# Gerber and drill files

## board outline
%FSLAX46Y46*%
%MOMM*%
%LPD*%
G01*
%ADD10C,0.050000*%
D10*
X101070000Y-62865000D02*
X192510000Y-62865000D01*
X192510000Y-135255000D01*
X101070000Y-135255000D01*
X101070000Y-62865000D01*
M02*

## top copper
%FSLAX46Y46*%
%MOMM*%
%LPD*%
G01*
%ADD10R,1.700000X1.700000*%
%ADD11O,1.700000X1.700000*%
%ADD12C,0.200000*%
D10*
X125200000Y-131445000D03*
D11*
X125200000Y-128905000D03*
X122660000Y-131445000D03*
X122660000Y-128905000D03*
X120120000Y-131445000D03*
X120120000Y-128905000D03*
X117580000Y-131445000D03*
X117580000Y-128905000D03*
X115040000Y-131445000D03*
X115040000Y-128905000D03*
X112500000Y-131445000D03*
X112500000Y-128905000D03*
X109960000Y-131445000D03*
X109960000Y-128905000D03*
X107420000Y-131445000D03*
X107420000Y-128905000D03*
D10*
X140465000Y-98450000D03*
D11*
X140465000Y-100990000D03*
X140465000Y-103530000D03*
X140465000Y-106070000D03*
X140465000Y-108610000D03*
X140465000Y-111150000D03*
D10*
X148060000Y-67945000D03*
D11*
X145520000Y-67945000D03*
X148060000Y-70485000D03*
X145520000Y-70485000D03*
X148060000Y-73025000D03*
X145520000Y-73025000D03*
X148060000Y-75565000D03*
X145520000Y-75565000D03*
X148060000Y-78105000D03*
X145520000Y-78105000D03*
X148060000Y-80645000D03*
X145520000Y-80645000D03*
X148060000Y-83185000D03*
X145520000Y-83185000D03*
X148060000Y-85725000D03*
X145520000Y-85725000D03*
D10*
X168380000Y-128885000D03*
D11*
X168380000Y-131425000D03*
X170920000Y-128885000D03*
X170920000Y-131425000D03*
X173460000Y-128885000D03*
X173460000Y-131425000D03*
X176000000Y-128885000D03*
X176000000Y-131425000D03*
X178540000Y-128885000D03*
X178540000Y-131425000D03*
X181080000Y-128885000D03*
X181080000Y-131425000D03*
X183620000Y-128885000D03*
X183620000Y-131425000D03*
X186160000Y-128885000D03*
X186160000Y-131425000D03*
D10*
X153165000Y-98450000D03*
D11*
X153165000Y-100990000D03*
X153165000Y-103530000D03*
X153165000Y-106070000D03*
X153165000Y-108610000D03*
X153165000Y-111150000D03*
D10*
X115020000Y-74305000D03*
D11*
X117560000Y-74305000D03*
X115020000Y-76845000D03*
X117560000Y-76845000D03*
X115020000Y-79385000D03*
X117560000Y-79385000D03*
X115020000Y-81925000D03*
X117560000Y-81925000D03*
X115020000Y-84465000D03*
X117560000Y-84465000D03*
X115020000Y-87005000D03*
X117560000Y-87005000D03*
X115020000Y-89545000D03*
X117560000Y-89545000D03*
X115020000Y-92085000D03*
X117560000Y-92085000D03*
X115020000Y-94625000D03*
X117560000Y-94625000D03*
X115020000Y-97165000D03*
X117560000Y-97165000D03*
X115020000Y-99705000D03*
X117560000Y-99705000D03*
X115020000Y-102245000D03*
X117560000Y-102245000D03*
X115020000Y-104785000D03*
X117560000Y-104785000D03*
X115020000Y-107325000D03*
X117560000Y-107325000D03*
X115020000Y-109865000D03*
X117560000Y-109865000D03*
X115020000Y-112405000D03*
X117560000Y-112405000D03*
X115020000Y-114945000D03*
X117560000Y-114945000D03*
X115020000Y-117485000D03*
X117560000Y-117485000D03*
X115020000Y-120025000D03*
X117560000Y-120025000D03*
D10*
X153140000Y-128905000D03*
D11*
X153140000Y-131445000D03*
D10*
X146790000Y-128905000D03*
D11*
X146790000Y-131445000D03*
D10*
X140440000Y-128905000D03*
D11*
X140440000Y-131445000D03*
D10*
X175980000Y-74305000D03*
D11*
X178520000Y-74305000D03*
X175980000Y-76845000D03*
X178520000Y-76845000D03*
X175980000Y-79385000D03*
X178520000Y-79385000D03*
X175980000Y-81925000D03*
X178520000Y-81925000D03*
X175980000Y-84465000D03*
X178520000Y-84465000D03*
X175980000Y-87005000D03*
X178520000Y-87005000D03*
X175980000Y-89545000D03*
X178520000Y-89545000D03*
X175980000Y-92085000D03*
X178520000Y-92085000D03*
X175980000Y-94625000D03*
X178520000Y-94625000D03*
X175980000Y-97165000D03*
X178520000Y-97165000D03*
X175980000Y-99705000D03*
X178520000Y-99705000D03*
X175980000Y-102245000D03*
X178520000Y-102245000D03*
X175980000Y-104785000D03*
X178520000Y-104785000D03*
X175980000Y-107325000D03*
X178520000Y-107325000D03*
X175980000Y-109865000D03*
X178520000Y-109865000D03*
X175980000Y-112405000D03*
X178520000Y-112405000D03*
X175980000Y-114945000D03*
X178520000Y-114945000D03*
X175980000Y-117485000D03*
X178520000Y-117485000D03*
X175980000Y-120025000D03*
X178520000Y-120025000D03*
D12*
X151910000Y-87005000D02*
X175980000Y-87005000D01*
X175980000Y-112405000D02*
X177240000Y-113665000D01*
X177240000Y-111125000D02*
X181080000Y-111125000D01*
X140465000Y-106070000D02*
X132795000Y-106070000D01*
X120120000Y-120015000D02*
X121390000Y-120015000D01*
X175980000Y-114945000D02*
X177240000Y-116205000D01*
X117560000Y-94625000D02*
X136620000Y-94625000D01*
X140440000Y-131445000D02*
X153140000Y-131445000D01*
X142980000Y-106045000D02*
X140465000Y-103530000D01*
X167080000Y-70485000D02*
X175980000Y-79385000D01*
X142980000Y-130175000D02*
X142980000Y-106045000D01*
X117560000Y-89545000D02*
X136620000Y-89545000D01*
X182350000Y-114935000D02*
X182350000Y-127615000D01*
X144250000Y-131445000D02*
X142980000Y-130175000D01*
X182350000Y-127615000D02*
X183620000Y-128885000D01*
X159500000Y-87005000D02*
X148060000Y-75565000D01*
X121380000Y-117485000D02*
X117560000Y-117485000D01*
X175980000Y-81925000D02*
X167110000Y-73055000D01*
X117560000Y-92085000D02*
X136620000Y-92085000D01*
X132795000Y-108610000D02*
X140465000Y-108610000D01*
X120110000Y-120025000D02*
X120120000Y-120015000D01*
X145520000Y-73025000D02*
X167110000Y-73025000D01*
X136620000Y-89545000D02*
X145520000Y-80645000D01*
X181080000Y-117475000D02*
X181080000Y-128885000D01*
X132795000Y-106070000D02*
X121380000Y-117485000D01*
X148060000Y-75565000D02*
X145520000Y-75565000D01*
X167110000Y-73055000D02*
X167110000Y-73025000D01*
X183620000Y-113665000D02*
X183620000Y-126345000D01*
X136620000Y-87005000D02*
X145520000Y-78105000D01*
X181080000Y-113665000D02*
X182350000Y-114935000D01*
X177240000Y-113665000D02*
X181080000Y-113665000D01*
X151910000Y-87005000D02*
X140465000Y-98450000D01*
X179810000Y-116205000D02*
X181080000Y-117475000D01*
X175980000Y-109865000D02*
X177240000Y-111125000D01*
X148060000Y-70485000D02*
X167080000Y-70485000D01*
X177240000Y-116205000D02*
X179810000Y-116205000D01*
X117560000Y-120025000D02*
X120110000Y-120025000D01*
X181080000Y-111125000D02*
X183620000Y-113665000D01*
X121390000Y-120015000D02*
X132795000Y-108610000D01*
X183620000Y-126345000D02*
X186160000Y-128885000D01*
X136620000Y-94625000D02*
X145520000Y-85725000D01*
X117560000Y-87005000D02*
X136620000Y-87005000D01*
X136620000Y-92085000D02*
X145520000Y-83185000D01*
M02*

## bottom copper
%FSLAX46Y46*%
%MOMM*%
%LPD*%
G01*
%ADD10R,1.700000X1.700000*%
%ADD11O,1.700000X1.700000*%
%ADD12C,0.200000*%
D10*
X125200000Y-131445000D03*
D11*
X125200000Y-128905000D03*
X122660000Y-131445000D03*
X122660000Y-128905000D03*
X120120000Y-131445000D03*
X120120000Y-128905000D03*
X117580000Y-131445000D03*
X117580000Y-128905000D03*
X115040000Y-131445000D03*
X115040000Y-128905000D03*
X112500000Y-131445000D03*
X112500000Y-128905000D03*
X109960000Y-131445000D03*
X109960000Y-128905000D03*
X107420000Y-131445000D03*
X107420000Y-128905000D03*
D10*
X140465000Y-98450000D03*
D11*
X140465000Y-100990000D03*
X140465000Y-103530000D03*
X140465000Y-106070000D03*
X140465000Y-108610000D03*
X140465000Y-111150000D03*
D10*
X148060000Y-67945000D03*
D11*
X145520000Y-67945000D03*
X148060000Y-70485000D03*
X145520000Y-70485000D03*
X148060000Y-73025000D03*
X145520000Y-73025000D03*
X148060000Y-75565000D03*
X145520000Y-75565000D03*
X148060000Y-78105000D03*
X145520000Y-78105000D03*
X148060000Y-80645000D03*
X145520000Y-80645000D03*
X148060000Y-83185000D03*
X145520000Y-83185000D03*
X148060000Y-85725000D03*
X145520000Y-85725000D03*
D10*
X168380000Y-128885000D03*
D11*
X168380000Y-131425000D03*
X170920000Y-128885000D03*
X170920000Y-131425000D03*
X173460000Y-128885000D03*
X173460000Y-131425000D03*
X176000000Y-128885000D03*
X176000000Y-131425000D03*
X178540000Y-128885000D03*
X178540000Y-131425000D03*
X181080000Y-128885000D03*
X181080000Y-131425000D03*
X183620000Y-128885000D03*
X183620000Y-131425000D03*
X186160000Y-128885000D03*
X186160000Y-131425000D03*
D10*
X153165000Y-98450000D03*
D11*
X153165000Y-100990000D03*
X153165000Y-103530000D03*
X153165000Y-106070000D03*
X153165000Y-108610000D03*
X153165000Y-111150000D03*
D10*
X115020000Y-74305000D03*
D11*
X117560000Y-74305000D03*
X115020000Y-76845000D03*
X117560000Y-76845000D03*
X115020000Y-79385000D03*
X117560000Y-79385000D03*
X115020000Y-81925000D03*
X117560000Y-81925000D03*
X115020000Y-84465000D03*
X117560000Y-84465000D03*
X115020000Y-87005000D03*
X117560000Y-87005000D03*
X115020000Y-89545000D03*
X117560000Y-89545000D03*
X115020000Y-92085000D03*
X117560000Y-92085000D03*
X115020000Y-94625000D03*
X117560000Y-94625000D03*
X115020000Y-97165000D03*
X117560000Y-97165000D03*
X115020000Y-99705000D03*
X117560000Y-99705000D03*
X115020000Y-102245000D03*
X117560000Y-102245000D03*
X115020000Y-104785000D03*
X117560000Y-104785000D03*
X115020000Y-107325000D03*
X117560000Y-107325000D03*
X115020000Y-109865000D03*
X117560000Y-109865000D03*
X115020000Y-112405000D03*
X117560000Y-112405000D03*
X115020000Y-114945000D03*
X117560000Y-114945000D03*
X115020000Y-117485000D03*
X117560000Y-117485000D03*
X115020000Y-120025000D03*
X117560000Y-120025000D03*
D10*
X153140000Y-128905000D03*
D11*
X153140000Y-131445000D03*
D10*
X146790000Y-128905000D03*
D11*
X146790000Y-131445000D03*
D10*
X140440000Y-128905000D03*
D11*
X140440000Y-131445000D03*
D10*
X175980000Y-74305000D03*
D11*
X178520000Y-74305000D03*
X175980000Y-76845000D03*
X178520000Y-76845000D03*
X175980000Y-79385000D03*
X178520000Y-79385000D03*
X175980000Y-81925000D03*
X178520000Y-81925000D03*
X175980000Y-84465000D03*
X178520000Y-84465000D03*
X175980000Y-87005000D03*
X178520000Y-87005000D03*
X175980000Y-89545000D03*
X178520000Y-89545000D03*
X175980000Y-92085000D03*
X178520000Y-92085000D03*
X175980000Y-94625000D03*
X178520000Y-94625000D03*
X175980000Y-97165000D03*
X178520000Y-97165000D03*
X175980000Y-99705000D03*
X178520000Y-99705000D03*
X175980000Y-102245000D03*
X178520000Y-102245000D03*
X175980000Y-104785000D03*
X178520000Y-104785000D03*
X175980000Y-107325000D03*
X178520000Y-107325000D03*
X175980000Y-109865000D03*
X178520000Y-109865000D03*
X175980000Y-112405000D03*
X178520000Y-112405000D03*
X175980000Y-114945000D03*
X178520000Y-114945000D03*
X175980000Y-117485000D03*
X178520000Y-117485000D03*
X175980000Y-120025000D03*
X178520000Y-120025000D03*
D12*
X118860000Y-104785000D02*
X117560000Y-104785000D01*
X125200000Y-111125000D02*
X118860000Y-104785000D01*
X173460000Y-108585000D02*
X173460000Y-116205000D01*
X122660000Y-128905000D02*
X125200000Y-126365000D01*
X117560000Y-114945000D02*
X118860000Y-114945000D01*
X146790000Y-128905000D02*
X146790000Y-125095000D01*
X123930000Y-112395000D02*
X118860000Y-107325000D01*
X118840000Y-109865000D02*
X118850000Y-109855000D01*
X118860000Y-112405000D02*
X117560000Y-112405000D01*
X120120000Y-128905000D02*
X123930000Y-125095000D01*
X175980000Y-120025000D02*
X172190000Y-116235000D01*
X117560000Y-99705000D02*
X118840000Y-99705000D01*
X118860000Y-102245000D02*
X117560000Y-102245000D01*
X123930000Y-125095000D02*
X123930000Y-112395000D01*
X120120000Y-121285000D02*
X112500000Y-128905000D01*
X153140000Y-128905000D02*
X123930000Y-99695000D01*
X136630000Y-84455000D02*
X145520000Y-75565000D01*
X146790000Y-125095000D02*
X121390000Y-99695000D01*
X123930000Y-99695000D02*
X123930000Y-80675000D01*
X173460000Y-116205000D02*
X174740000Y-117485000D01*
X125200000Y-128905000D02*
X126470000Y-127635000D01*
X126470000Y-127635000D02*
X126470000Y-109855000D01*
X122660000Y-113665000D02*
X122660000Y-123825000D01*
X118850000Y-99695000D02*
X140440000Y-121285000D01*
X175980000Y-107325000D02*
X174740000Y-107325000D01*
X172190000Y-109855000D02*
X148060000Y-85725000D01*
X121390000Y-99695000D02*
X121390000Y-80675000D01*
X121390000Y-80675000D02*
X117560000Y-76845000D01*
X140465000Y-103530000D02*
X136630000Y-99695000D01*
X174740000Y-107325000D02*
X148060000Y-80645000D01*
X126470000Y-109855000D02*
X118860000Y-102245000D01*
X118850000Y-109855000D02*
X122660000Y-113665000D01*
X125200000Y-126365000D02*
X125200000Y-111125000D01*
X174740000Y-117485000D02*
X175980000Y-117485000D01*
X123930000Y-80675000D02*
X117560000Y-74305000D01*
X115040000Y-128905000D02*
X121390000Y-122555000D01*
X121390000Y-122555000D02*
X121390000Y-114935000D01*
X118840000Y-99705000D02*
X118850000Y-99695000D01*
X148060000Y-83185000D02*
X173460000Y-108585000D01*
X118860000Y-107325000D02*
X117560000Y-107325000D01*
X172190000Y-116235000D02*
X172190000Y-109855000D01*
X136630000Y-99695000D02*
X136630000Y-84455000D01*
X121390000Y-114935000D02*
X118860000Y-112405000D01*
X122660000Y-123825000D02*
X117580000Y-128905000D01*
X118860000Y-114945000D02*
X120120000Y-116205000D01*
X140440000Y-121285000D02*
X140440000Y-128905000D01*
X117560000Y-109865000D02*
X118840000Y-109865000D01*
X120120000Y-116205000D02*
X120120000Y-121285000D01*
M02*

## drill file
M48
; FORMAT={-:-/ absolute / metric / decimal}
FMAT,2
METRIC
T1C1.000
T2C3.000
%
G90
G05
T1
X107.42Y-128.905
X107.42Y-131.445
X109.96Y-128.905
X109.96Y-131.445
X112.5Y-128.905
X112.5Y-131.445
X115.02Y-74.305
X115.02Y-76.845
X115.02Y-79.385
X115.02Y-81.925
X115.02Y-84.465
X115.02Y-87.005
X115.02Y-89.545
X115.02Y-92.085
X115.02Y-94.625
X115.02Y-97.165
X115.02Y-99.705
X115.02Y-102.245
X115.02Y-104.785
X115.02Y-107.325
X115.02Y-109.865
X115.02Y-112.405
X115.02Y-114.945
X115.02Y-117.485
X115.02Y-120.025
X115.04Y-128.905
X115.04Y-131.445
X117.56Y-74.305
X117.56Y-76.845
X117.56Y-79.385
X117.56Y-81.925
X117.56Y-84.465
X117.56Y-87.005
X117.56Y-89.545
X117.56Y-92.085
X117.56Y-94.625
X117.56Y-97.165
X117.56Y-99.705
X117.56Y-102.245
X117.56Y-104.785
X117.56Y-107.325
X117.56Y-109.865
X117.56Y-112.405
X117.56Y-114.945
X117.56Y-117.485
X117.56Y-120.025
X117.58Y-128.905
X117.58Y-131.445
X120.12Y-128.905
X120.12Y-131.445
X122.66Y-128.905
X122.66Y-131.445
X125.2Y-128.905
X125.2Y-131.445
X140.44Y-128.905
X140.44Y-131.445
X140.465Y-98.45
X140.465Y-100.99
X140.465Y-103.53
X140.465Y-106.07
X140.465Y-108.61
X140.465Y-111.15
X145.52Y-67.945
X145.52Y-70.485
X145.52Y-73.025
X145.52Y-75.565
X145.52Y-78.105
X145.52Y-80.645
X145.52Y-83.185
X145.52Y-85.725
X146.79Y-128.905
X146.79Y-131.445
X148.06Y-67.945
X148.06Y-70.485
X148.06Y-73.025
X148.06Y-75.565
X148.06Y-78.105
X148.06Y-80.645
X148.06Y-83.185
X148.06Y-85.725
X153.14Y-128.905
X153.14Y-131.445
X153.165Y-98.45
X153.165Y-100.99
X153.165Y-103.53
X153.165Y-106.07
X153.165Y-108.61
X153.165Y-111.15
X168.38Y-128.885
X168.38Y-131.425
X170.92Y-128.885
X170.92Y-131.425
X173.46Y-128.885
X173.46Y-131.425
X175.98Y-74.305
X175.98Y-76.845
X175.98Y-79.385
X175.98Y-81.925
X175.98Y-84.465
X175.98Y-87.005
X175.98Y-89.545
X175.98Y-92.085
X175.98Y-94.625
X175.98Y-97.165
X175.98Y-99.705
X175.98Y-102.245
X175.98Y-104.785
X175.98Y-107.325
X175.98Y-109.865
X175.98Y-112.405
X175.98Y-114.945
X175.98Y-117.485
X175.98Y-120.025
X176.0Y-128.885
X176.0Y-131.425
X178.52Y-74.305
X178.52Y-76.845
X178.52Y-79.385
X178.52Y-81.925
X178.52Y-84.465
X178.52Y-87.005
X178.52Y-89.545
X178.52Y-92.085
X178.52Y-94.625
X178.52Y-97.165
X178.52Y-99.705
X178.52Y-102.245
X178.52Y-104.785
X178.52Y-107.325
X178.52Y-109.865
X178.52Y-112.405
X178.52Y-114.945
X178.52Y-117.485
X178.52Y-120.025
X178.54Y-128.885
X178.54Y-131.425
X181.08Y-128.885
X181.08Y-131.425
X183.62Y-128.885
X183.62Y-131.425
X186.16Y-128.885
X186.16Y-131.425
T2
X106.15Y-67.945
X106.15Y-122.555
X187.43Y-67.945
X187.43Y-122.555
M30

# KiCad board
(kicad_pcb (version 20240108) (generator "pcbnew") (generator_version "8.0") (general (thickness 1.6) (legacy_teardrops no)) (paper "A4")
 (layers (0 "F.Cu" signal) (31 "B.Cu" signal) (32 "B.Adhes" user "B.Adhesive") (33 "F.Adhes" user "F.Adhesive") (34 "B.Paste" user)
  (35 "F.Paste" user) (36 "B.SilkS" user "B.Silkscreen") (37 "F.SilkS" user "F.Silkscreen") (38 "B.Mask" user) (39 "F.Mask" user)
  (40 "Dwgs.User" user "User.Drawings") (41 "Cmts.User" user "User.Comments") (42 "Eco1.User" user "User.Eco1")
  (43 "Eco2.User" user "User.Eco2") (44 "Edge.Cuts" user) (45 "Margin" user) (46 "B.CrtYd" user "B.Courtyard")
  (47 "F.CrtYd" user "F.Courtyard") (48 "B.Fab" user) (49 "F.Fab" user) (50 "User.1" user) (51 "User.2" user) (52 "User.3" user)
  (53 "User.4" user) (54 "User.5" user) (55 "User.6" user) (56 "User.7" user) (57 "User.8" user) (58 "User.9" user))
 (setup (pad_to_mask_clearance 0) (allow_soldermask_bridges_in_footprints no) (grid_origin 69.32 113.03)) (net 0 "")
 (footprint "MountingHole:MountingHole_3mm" (layer "F.Cu") (at 106.15 67.945)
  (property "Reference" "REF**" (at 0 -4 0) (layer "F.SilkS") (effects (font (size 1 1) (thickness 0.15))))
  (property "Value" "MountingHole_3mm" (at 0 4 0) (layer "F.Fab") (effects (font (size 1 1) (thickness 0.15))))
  (pad "" np_thru_hole circle (at 0 0) (size 3 3) (drill 3) (layers "*.Cu" "*.Mask")))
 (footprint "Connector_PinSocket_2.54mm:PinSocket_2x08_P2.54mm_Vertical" (layer "F.Cu") (at 125.2 131.445 -90)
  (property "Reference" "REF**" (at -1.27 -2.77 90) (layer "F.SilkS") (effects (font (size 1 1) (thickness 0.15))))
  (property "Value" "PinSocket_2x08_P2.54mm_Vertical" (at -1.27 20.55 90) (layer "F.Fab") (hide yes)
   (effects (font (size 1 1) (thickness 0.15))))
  (pad "1" thru_hole rect (at 0 0 270) (size 1.7 1.7) (drill 1) (layers "*.Cu" "*.Mask") (remove_unused_layers no))
  (pad "2" thru_hole oval (at -2.54 0 270) (size 1.7 1.7) (drill 1) (layers "*.Cu" "*.Mask") (remove_unused_layers no))
  (pad "3" thru_hole oval (at 0 2.54 270) (size 1.7 1.7) (drill 1) (layers "*.Cu" "*.Mask") (remove_unused_layers no))
  (pad "4" thru_hole oval (at -2.54 2.54 270) (size 1.7 1.7) (drill 1) (layers "*.Cu" "*.Mask") (remove_unused_layers no))
  (pad "5" thru_hole oval (at 0 5.08 270) (size 1.7 1.7) (drill 1) (layers "*.Cu" "*.Mask") (remove_unused_layers no))
  (pad "6" thru_hole oval (at -2.54 5.08 270) (size 1.7 1.7) (drill 1) (layers "*.Cu" "*.Mask") (remove_unused_layers no))
  (pad "7" thru_hole oval (at 0 7.62 270) (size 1.7 1.7) (drill 1) (layers "*.Cu" "*.Mask") (remove_unused_layers no))
  (pad "8" thru_hole oval (at -2.54 7.62 270) (size 1.7 1.7) (drill 1) (layers "*.Cu" "*.Mask") (remove_unused_layers no))
  (pad "9" thru_hole oval (at 0 10.16 270) (size 1.7 1.7) (drill 1) (layers "*.Cu" "*.Mask") (remove_unused_layers no))
  (pad "10" thru_hole oval (at -2.54 10.16 270) (size 1.7 1.7) (drill 1) (layers "*.Cu" "*.Mask") (remove_unused_layers no))
  (pad "11" thru_hole oval (at 0 12.7 270) (size 1.7 1.7) (drill 1) (layers "*.Cu" "*.Mask") (remove_unused_layers no))
  (pad "12" thru_hole oval (at -2.54 12.7 270) (size 1.7 1.7) (drill 1) (layers "*.Cu" "*.Mask") (remove_unused_layers no))
  (pad "13" thru_hole oval (at 0 15.24 270) (size 1.7 1.7) (drill 1) (layers "*.Cu" "*.Mask") (remove_unused_layers no))
  (pad "14" thru_hole oval (at -2.54 15.24 270) (size 1.7 1.7) (drill 1) (layers "*.Cu" "*.Mask") (remove_unused_layers no))
  (pad "15" thru_hole oval (at 0 17.78 270) (size 1.7 1.7) (drill 1) (layers "*.Cu" "*.Mask") (remove_unused_layers no))
  (pad "16" thru_hole oval (at -2.54 17.78 270) (size 1.7 1.7) (drill 1) (layers "*.Cu" "*.Mask") (remove_unused_layers no)))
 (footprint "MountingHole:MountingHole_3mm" (layer "F.Cu") (at 187.43 122.555)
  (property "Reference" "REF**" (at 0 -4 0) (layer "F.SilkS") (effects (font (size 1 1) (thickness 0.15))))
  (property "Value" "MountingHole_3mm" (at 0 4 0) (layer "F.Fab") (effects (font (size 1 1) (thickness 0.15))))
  (pad "" np_thru_hole circle (at 0 0) (size 3 3) (drill 3) (layers "*.Cu" "*.Mask")))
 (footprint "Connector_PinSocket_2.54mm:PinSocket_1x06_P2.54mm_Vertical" (layer "F.Cu") (at 140.465 98.45)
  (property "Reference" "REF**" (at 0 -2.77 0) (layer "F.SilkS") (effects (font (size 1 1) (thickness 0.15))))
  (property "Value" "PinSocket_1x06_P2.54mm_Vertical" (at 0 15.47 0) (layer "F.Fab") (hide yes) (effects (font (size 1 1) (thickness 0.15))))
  (pad "1" thru_hole rect (at 0 0) (size 1.7 1.7) (drill 1) (layers "*.Cu" "*.Mask") (remove_unused_layers no))
  (pad "2" thru_hole oval (at 0 2.54) (size 1.7 1.7) (drill 1) (layers "*.Cu" "*.Mask") (remove_unused_layers no))
  (pad "3" thru_hole oval (at 0 5.08) (size 1.7 1.7) (drill 1) (layers "*.Cu" "*.Mask") (remove_unused_layers no))
  (pad "4" thru_hole oval (at 0 7.62) (size 1.7 1.7) (drill 1) (layers "*.Cu" "*.Mask") (remove_unused_layers no))
  (pad "5" thru_hole oval (at 0 10.16) (size 1.7 1.7) (drill 1) (layers "*.Cu" "*.Mask") (remove_unused_layers no))
  (pad "6" thru_hole oval (at 0 12.7) (size 1.7 1.7) (drill 1) (layers "*.Cu" "*.Mask") (remove_unused_layers no)))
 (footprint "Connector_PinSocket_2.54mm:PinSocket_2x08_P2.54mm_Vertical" (layer "F.Cu") (at 148.06 67.945)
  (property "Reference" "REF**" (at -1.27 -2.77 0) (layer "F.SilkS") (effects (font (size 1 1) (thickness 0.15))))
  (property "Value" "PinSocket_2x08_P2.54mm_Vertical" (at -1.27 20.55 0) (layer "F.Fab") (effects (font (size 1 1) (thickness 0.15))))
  (pad "1" thru_hole rect (at 0 0) (size 1.7 1.7) (drill 1) (layers "*.Cu" "*.Mask") (remove_unused_layers no))
  (pad "2" thru_hole oval (at -2.54 0) (size 1.7 1.7) (drill 1) (layers "*.Cu" "*.Mask") (remove_unused_layers no))
  (pad "3" thru_hole oval (at 0 2.54) (size 1.7 1.7) (drill 1) (layers "*.Cu" "*.Mask") (remove_unused_layers no))
  (pad "4" thru_hole oval (at -2.54 2.54) (size 1.7 1.7) (drill 1) (layers "*.Cu" "*.Mask") (remove_unused_layers no))
  (pad "5" thru_hole oval (at 0 5.08) (size 1.7 1.7) (drill 1) (layers "*.Cu" "*.Mask") (remove_unused_layers no))
  (pad "6" thru_hole oval (at -2.54 5.08) (size 1.7 1.7) (drill 1) (layers "*.Cu" "*.Mask") (remove_unused_layers no))
  (pad "7" thru_hole oval (at 0 7.62) (size 1.7 1.7) (drill 1) (layers "*.Cu" "*.Mask") (remove_unused_layers no))
  (pad "8" thru_hole oval (at -2.54 7.62) (size 1.7 1.7) (drill 1) (layers "*.Cu" "*.Mask") (remove_unused_layers no))
  (pad "9" thru_hole oval (at 0 10.16) (size 1.7 1.7) (drill 1) (layers "*.Cu" "*.Mask") (remove_unused_layers no))
  (pad "10" thru_hole oval (at -2.54 10.16) (size 1.7 1.7) (drill 1) (layers "*.Cu" "*.Mask") (remove_unused_layers no))
  (pad "11" thru_hole oval (at 0 12.7) (size 1.7 1.7) (drill 1) (layers "*.Cu" "*.Mask") (remove_unused_layers no))
  (pad "12" thru_hole oval (at -2.54 12.7) (size 1.7 1.7) (drill 1) (layers "*.Cu" "*.Mask") (remove_unused_layers no))
  (pad "13" thru_hole oval (at 0 15.24) (size 1.7 1.7) (drill 1) (layers "*.Cu" "*.Mask") (remove_unused_layers no))
  (pad "14" thru_hole oval (at -2.54 15.24) (size 1.7 1.7) (drill 1) (layers "*.Cu" "*.Mask") (remove_unused_layers no))
  (pad "15" thru_hole oval (at 0 17.78) (size 1.7 1.7) (drill 1) (layers "*.Cu" "*.Mask") (remove_unused_layers no))
  (pad "16" thru_hole oval (at -2.54 17.78) (size 1.7 1.7) (drill 1) (layers "*.Cu" "*.Mask") (remove_unused_layers no)))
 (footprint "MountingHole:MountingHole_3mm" (layer "F.Cu") (at 106.15 122.555)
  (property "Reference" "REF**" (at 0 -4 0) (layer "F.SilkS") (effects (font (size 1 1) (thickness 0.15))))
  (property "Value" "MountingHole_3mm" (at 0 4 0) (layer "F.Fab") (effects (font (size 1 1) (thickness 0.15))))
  (pad "" np_thru_hole circle (at 0 0) (size 3 3) (drill 3) (layers "*.Cu" "*.Mask")))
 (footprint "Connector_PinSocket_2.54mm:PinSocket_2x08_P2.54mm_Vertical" (layer "F.Cu") (at 168.38 128.885 90)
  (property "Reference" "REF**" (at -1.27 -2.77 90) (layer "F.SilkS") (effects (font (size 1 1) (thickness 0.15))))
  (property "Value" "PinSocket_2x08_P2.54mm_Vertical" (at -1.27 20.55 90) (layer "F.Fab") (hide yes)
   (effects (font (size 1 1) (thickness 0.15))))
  (pad "1" thru_hole rect (at 0 0 90) (size 1.7 1.7) (drill 1) (layers "*.Cu" "*.Mask") (remove_unused_layers no))
  (pad "2" thru_hole oval (at -2.54 0 90) (size 1.7 1.7) (drill 1) (layers "*.Cu" "*.Mask") (remove_unused_layers no))
  (pad "3" thru_hole oval (at 0 2.54 90) (size 1.7 1.7) (drill 1) (layers "*.Cu" "*.Mask") (remove_unused_layers no))
  (pad "4" thru_hole oval (at -2.54 2.54 90) (size 1.7 1.7) (drill 1) (layers "*.Cu" "*.Mask") (remove_unused_layers no))
  (pad "5" thru_hole oval (at 0 5.08 90) (size 1.7 1.7) (drill 1) (layers "*.Cu" "*.Mask") (remove_unused_layers no))
  (pad "6" thru_hole oval (at -2.54 5.08 90) (size 1.7 1.7) (drill 1) (layers "*.Cu" "*.Mask") (remove_unused_layers no))
  (pad "7" thru_hole oval (at 0 7.62 90) (size 1.7 1.7) (drill 1) (layers "*.Cu" "*.Mask") (remove_unused_layers no))
  (pad "8" thru_hole oval (at -2.54 7.62 90) (size 1.7 1.7) (drill 1) (layers "*.Cu" "*.Mask") (remove_unused_layers no))
  (pad "9" thru_hole oval (at 0 10.16 90) (size 1.7 1.7) (drill 1) (layers "*.Cu" "*.Mask") (remove_unused_layers no))
  (pad "10" thru_hole oval (at -2.54 10.16 90) (size 1.7 1.7) (drill 1) (layers "*.Cu" "*.Mask") (remove_unused_layers no))
  (pad "11" thru_hole oval (at 0 12.7 90) (size 1.7 1.7) (drill 1) (layers "*.Cu" "*.Mask") (remove_unused_layers no))
  (pad "12" thru_hole oval (at -2.54 12.7 90) (size 1.7 1.7) (drill 1) (layers "*.Cu" "*.Mask") (remove_unused_layers no))
  (pad "13" thru_hole oval (at 0 15.24 90) (size 1.7 1.7) (drill 1) (layers "*.Cu" "*.Mask") (remove_unused_layers no))
  (pad "14" thru_hole oval (at -2.54 15.24 90) (size 1.7 1.7) (drill 1) (layers "*.Cu" "*.Mask") (remove_unused_layers no))
  (pad "15" thru_hole oval (at 0 17.78 90) (size 1.7 1.7) (drill 1) (layers "*.Cu" "*.Mask") (remove_unused_layers no))
  (pad "16" thru_hole oval (at -2.54 17.78 90) (size 1.7 1.7) (drill 1) (layers "*.Cu" "*.Mask") (remove_unused_layers no)))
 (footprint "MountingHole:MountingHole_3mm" (layer "F.Cu") (at 187.43 67.945)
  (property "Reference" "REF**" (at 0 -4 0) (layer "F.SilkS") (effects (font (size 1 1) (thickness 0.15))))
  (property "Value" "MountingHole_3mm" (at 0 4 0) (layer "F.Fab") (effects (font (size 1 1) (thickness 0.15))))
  (pad "" np_thru_hole circle (at 0 0) (size 3 3) (drill 3) (layers "*.Cu" "*.Mask")))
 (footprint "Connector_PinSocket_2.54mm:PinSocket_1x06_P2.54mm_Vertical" (layer "F.Cu") (at 153.165 98.45)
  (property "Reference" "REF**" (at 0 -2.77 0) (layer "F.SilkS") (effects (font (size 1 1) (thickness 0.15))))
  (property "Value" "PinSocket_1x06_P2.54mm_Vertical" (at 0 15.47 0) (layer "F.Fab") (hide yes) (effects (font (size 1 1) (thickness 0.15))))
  (pad "1" thru_hole rect (at 0 0) (size 1.7 1.7) (drill 1) (layers "*.Cu" "*.Mask") (remove_unused_layers no))
  (pad "2" thru_hole oval (at 0 2.54) (size 1.7 1.7) (drill 1) (layers "*.Cu" "*.Mask") (remove_unused_layers no))
  (pad "3" thru_hole oval (at 0 5.08) (size 1.7 1.7) (drill 1) (layers "*.Cu" "*.Mask") (remove_unused_layers no))
  (pad "4" thru_hole oval (at 0 7.62) (size 1.7 1.7) (drill 1) (layers "*.Cu" "*.Mask") (remove_unused_layers no))
  (pad "5" thru_hole oval (at 0 10.16) (size 1.7 1.7) (drill 1) (layers "*.Cu" "*.Mask") (remove_unused_layers no))
  (pad "6" thru_hole oval (at 0 12.7) (size 1.7 1.7) (drill 1) (layers "*.Cu" "*.Mask") (remove_unused_layers no)))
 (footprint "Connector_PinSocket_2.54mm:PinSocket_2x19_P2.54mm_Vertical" (layer "B.Cu") (at 115.02 74.305 180)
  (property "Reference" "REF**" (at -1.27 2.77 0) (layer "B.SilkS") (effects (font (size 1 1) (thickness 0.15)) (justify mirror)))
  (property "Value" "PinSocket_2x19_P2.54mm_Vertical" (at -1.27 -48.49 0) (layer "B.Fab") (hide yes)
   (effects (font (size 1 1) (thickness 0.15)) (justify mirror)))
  (pad "1" thru_hole rect (at 0 0 180) (size 1.7 1.7) (drill 1) (layers "*.Cu" "*.Mask") (remove_unused_layers no))
  (pad "2" thru_hole oval (at -2.54 0 180) (size 1.7 1.7) (drill 1) (layers "*.Cu" "*.Mask") (remove_unused_layers no))
  (pad "3" thru_hole oval (at 0 -2.54 180) (size 1.7 1.7) (drill 1) (layers "*.Cu" "*.Mask") (remove_unused_layers no))
  (pad "4" thru_hole oval (at -2.54 -2.54 180) (size 1.7 1.7) (drill 1) (layers "*.Cu" "*.Mask") (remove_unused_layers no))
  (pad "5" thru_hole oval (at 0 -5.08 180) (size 1.7 1.7) (drill 1) (layers "*.Cu" "*.Mask") (remove_unused_layers no))
  (pad "6" thru_hole oval (at -2.54 -5.08 180) (size 1.7 1.7) (drill 1) (layers "*.Cu" "*.Mask") (remove_unused_layers no))
  (pad "7" thru_hole oval (at 0 -7.62 180) (size 1.7 1.7) (drill 1) (layers "*.Cu" "*.Mask") (remove_unused_layers no))
  (pad "8" thru_hole oval (at -2.54 -7.62 180) (size 1.7 1.7) (drill 1) (layers "*.Cu" "*.Mask") (remove_unused_layers no))
  (pad "9" thru_hole oval (at 0 -10.16 180) (size 1.7 1.7) (drill 1) (layers "*.Cu" "*.Mask") (remove_unused_layers no))
  (pad "10" thru_hole oval (at -2.54 -10.16 180) (size 1.7 1.7) (drill 1) (layers "*.Cu" "*.Mask") (remove_unused_layers no))
  (pad "11" thru_hole oval (at 0 -12.7 180) (size 1.7 1.7) (drill 1) (layers "*.Cu" "*.Mask") (remove_unused_layers no))
  (pad "12" thru_hole oval (at -2.54 -12.7 180) (size 1.7 1.7) (drill 1) (layers "*.Cu" "*.Mask") (remove_unused_layers no))
  (pad "13" thru_hole oval (at 0 -15.24 180) (size 1.7 1.7) (drill 1) (layers "*.Cu" "*.Mask") (remove_unused_layers no))
  (pad "14" thru_hole oval (at -2.54 -15.24 180) (size 1.7 1.7) (drill 1) (layers "*.Cu" "*.Mask") (remove_unused_layers no))
  (pad "15" thru_hole oval (at 0 -17.78 180) (size 1.7 1.7) (drill 1) (layers "*.Cu" "*.Mask") (remove_unused_layers no))
  (pad "16" thru_hole oval (at -2.54 -17.78 180) (size 1.7 1.7) (drill 1) (layers "*.Cu" "*.Mask") (remove_unused_layers no))
  (pad "17" thru_hole oval (at 0 -20.32 180) (size 1.7 1.7) (drill 1) (layers "*.Cu" "*.Mask") (remove_unused_layers no))
  (pad "18" thru_hole oval (at -2.54 -20.32 180) (size 1.7 1.7) (drill 1) (layers "*.Cu" "*.Mask") (remove_unused_layers no))
  (pad "19" thru_hole oval (at 0 -22.86 180) (size 1.7 1.7) (drill 1) (layers "*.Cu" "*.Mask") (remove_unused_layers no))
  (pad "20" thru_hole oval (at -2.54 -22.86 180) (size 1.7 1.7) (drill 1) (layers "*.Cu" "*.Mask") (remove_unused_layers no))
  (pad "21" thru_hole oval (at 0 -25.4 180) (size 1.7 1.7) (drill 1) (layers "*.Cu" "*.Mask") (remove_unused_layers no))
  (pad "22" thru_hole oval (at -2.54 -25.4 180) (size 1.7 1.7) (drill 1) (layers "*.Cu" "*.Mask") (remove_unused_layers no))
  (pad "23" thru_hole oval (at 0 -27.94 180) (size 1.7 1.7) (drill 1) (layers "*.Cu" "*.Mask") (remove_unused_layers no))
  (pad "24" thru_hole oval (at -2.54 -27.94 180) (size 1.7 1.7) (drill 1) (layers "*.Cu" "*.Mask") (remove_unused_layers no))
  (pad "25" thru_hole oval (at 0 -30.48 180) (size 1.7 1.7) (drill 1) (layers "*.Cu" "*.Mask") (remove_unused_layers no))
  (pad "26" thru_hole oval (at -2.54 -30.48 180) (size 1.7 1.7) (drill 1) (layers "*.Cu" "*.Mask") (remove_unused_layers no))
  (pad "27" thru_hole oval (at 0 -33.02 180) (size 1.7 1.7) (drill 1) (layers "*.Cu" "*.Mask") (remove_unused_layers no))
  (pad "28" thru_hole oval (at -2.54 -33.02 180) (size 1.7 1.7) (drill 1) (layers "*.Cu" "*.Mask") (remove_unused_layers no))
  (pad "29" thru_hole oval (at 0 -35.56 180) (size 1.7 1.7) (drill 1) (layers "*.Cu" "*.Mask") (remove_unused_layers no))
  (pad "30" thru_hole oval (at -2.54 -35.56 180) (size 1.7 1.7) (drill 1) (layers "*.Cu" "*.Mask") (remove_unused_layers no))
  (pad "31" thru_hole oval (at 0 -38.1 180) (size 1.7 1.7) (drill 1) (layers "*.Cu" "*.Mask") (remove_unused_layers no))
  (pad "32" thru_hole oval (at -2.54 -38.1 180) (size 1.7 1.7) (drill 1) (layers "*.Cu" "*.Mask") (remove_unused_layers no))
  (pad "33" thru_hole oval (at 0 -40.64 180) (size 1.7 1.7) (drill 1) (layers "*.Cu" "*.Mask") (remove_unused_layers no))
  (pad "34" thru_hole oval (at -2.54 -40.64 180) (size 1.7 1.7) (drill 1) (layers "*.Cu" "*.Mask") (remove_unused_layers no))
  (pad "35" thru_hole oval (at 0 -43.18 180) (size 1.7 1.7) (drill 1) (layers "*.Cu" "*.Mask") (remove_unused_layers no))
  (pad "36" thru_hole oval (at -2.54 -43.18 180) (size 1.7 1.7) (drill 1) (layers "*.Cu" "*.Mask") (remove_unused_layers no))
  (pad "37" thru_hole oval (at 0 -45.72 180) (size 1.7 1.7) (drill 1) (layers "*.Cu" "*.Mask") (remove_unused_layers no))
  (pad "38" thru_hole oval (at -2.54 -45.72 180) (size 1.7 1.7) (drill 1) (layers "*.Cu" "*.Mask") (remove_unused_layers no)))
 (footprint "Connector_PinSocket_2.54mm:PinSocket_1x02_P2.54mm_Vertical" (layer "B.Cu") (at 153.14 128.905 180)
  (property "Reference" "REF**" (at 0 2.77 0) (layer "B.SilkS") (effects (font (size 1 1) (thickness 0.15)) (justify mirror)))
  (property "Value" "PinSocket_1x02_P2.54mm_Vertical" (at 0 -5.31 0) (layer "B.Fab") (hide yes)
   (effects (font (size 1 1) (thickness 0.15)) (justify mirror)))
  (pad "1" thru_hole rect (at 0 0 180) (size 1.7 1.7) (drill 1) (layers "*.Cu" "*.Mask") (remove_unused_layers no))
  (pad "2" thru_hole oval (at 0 -2.54 180) (size 1.7 1.7) (drill 1) (layers "*.Cu" "*.Mask") (remove_unused_layers no)))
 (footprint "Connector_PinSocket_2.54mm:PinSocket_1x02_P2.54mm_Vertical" (layer "B.Cu") (at 146.79 128.905 180)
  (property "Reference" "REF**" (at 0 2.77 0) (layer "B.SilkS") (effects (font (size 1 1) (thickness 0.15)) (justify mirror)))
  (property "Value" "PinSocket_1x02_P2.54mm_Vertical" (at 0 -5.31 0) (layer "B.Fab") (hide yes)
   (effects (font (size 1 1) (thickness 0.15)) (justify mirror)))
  (pad "1" thru_hole rect (at 0 0 180) (size 1.7 1.7) (drill 1) (layers "*.Cu" "*.Mask") (remove_unused_layers no))
  (pad "2" thru_hole oval (at 0 -2.54 180) (size 1.7 1.7) (drill 1) (layers "*.Cu" "*.Mask") (remove_unused_layers no)))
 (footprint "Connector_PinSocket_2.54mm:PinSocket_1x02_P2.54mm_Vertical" (layer "B.Cu") (at 140.44 128.905 180)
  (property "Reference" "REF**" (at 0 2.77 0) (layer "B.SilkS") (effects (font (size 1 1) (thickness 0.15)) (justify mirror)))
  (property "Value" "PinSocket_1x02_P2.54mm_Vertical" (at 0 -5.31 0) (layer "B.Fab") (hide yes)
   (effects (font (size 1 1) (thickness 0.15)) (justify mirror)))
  (pad "1" thru_hole rect (at 0 0 180) (size 1.7 1.7) (drill 1) (layers "*.Cu" "*.Mask") (remove_unused_layers no))
  (pad "2" thru_hole oval (at 0 -2.54 180) (size 1.7 1.7) (drill 1) (layers "*.Cu" "*.Mask") (remove_unused_layers no)))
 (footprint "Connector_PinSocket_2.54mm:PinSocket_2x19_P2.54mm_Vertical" (layer "B.Cu") (at 175.98 74.305 180)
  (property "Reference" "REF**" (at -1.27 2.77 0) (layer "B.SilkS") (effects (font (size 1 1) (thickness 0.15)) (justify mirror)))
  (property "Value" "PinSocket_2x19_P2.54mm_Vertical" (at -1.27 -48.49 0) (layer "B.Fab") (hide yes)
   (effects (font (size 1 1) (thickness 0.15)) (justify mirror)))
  (pad "1" thru_hole rect (at 0 0 180) (size 1.7 1.7) (drill 1) (layers "*.Cu" "*.Mask") (remove_unused_layers no))
  (pad "2" thru_hole oval (at -2.54 0 180) (size 1.7 1.7) (drill 1) (layers "*.Cu" "*.Mask") (remove_unused_layers no))
  (pad "3" thru_hole oval (at 0 -2.54 180) (size 1.7 1.7) (drill 1) (layers "*.Cu" "*.Mask") (remove_unused_layers no))
  (pad "4" thru_hole oval (at -2.54 -2.54 180) (size 1.7 1.7) (drill 1) (layers "*.Cu" "*.Mask") (remove_unused_layers no))
  (pad "5" thru_hole oval (at 0 -5.08 180) (size 1.7 1.7) (drill 1) (layers "*.Cu" "*.Mask") (remove_unused_layers no))
  (pad "6" thru_hole oval (at -2.54 -5.08 180) (size 1.7 1.7) (drill 1) (layers "*.Cu" "*.Mask") (remove_unused_layers no))
  (pad "7" thru_hole oval (at 0 -7.62 180) (size 1.7 1.7) (drill 1) (layers "*.Cu" "*.Mask") (remove_unused_layers no))
  (pad "8" thru_hole oval (at -2.54 -7.62 180) (size 1.7 1.7) (drill 1) (layers "*.Cu" "*.Mask") (remove_unused_layers no))
  (pad "9" thru_hole oval (at 0 -10.16 180) (size 1.7 1.7) (drill 1) (layers "*.Cu" "*.Mask") (remove_unused_layers no))
  (pad "10" thru_hole oval (at -2.54 -10.16 180) (size 1.7 1.7) (drill 1) (layers "*.Cu" "*.Mask") (remove_unused_layers no))
  (pad "11" thru_hole oval (at 0 -12.7 180) (size 1.7 1.7) (drill 1) (layers "*.Cu" "*.Mask") (remove_unused_layers no))
  (pad "12" thru_hole oval (at -2.54 -12.7 180) (size 1.7 1.7) (drill 1) (layers "*.Cu" "*.Mask") (remove_unused_layers no))
  (pad "13" thru_hole oval (at 0 -15.24 180) (size 1.7 1.7) (drill 1) (layers "*.Cu" "*.Mask") (remove_unused_layers no))
  (pad "14" thru_hole oval (at -2.54 -15.24 180) (size 1.7 1.7) (drill 1) (layers "*.Cu" "*.Mask") (remove_unused_layers no))
  (pad "15" thru_hole oval (at 0 -17.78 180) (size 1.7 1.7) (drill 1) (layers "*.Cu" "*.Mask") (remove_unused_layers no))
  (pad "16" thru_hole oval (at -2.54 -17.78 180) (size 1.7 1.7) (drill 1) (layers "*.Cu" "*.Mask") (remove_unused_layers no))
  (pad "17" thru_hole oval (at 0 -20.32 180) (size 1.7 1.7) (drill 1) (layers "*.Cu" "*.Mask") (remove_unused_layers no))
  (pad "18" thru_hole oval (at -2.54 -20.32 180) (size 1.7 1.7) (drill 1) (layers "*.Cu" "*.Mask") (remove_unused_layers no))
  (pad "19" thru_hole oval (at 0 -22.86 180) (size 1.7 1.7) (drill 1) (layers "*.Cu" "*.Mask") (remove_unused_layers no))
  (pad "20" thru_hole oval (at -2.54 -22.86 180) (size 1.7 1.7) (drill 1) (layers "*.Cu" "*.Mask") (remove_unused_layers no))
  (pad "21" thru_hole oval (at 0 -25.4 180) (size 1.7 1.7) (drill 1) (layers "*.Cu" "*.Mask") (remove_unused_layers no))
  (pad "22" thru_hole oval (at -2.54 -25.4 180) (size 1.7 1.7) (drill 1) (layers "*.Cu" "*.Mask") (remove_unused_layers no))
  (pad "23" thru_hole oval (at 0 -27.94 180) (size 1.7 1.7) (drill 1) (layers "*.Cu" "*.Mask") (remove_unused_layers no))
  (pad "24" thru_hole oval (at -2.54 -27.94 180) (size 1.7 1.7) (drill 1) (layers "*.Cu" "*.Mask") (remove_unused_layers no))
  (pad "25" thru_hole oval (at 0 -30.48 180) (size 1.7 1.7) (drill 1) (layers "*.Cu" "*.Mask") (remove_unused_layers no))
  (pad "26" thru_hole oval (at -2.54 -30.48 180) (size 1.7 1.7) (drill 1) (layers "*.Cu" "*.Mask") (remove_unused_layers no))
  (pad "27" thru_hole oval (at 0 -33.02 180) (size 1.7 1.7) (drill 1) (layers "*.Cu" "*.Mask") (remove_unused_layers no))
  (pad "28" thru_hole oval (at -2.54 -33.02 180) (size 1.7 1.7) (drill 1) (layers "*.Cu" "*.Mask") (remove_unused_layers no))
  (pad "29" thru_hole oval (at 0 -35.56 180) (size 1.7 1.7) (drill 1) (layers "*.Cu" "*.Mask") (remove_unused_layers no))
  (pad "30" thru_hole oval (at -2.54 -35.56 180) (size 1.7 1.7) (drill 1) (layers "*.Cu" "*.Mask") (remove_unused_layers no))
  (pad "31" thru_hole oval (at 0 -38.1 180) (size 1.7 1.7) (drill 1) (layers "*.Cu" "*.Mask") (remove_unused_layers no))
  (pad "32" thru_hole oval (at -2.54 -38.1 180) (size 1.7 1.7) (drill 1) (layers "*.Cu" "*.Mask") (remove_unused_layers no))
  (pad "33" thru_hole oval (at 0 -40.64 180) (size 1.7 1.7) (drill 1) (layers "*.Cu" "*.Mask") (remove_unused_layers no))
  (pad "34" thru_hole oval (at -2.54 -40.64 180) (size 1.7 1.7) (drill 1) (layers "*.Cu" "*.Mask") (remove_unused_layers no))
  (pad "35" thru_hole oval (at 0 -43.18 180) (size 1.7 1.7) (drill 1) (layers "*.Cu" "*.Mask") (remove_unused_layers no))
  (pad "36" thru_hole oval (at -2.54 -43.18 180) (size 1.7 1.7) (drill 1) (layers "*.Cu" "*.Mask") (remove_unused_layers no))
  (pad "37" thru_hole oval (at 0 -45.72 180) (size 1.7 1.7) (drill 1) (layers "*.Cu" "*.Mask") (remove_unused_layers no))
  (pad "38" thru_hole oval (at -2.54 -45.72 180) (size 1.7 1.7) (drill 1) (layers "*.Cu" "*.Mask") (remove_unused_layers no)))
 (gr_rect (start 101.07 62.865) (end 192.51 135.255) (stroke (width 0.05) (type default)) (fill none) (layer "Edge.Cuts"))
 (segment (start 151.91 87.005) (end 175.98 87.005) (width 0.2) (layer "F.Cu") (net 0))
 (segment (start 175.98 112.405) (end 177.24 113.665) (width 0.2) (layer "F.Cu") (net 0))
 (segment (start 177.24 111.125) (end 181.08 111.125) (width 0.2) (layer "F.Cu") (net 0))
 (segment (start 140.465 106.07) (end 132.795 106.07) (width 0.2) (layer "F.Cu") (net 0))
 (segment (start 120.12 120.015) (end 121.39 120.015) (width 0.2) (layer "F.Cu") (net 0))
 (segment (start 175.98 114.945) (end 177.24 116.205) (width 0.2) (layer "F.Cu") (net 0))
 (segment (start 117.56 94.625) (end 136.62 94.625) (width 0.2) (layer "F.Cu") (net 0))
 (segment (start 140.44 131.445) (end 153.14 131.445) (width 0.2) (layer "F.Cu") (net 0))
 (segment (start 142.98 106.045) (end 140.465 103.53) (width 0.2) (layer "F.Cu") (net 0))
 (segment (start 167.08 70.485) (end 175.98 79.385) (width 0.2) (layer "F.Cu") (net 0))
 (segment (start 142.98 130.175) (end 142.98 106.045) (width 0.2) (layer "F.Cu") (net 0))
 (segment (start 117.56 89.545) (end 136.62 89.545) (width 0.2) (layer "F.Cu") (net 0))
 (segment (start 182.35 114.935) (end 182.35 127.615) (width 0.2) (layer "F.Cu") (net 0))
 (segment (start 144.25 131.445) (end 142.98 130.175) (width 0.2) (layer "F.Cu") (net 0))
 (segment (start 182.35 127.615) (end 183.62 128.885) (width 0.2) (layer "F.Cu") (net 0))
 (segment (start 159.5 87.005) (end 148.06 75.565) (width 0.2) (layer "F.Cu") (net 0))
 (segment (start 121.38 117.485) (end 117.56 117.485) (width 0.2) (layer "F.Cu") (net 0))
 (segment (start 175.98 81.925) (end 167.11 73.055) (width 0.2) (layer "F.Cu") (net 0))
 (segment (start 117.56 92.085) (end 136.62 92.085) (width 0.2) (layer "F.Cu") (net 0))
 (segment (start 132.795 108.61) (end 140.465 108.61) (width 0.2) (layer "F.Cu") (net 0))
 (segment (start 120.11 120.025) (end 120.12 120.015) (width 0.2) (layer "F.Cu") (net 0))
 (segment (start 145.52 73.025) (end 167.11 73.025) (width 0.2) (layer "F.Cu") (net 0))
 (segment (start 136.62 89.545) (end 145.52 80.645) (width 0.2) (layer "F.Cu") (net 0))
 (segment (start 181.08 117.475) (end 181.08 128.885) (width 0.2) (layer "F.Cu") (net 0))
 (segment (start 132.795 106.07) (end 121.38 117.485) (width 0.2) (layer "F.Cu") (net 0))
 (segment (start 148.06 75.565) (end 145.52 75.565) (width 0.2) (layer "F.Cu") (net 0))
 (segment (start 167.11 73.055) (end 167.11 73.025) (width 0.2) (layer "F.Cu") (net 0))
 (segment (start 183.62 113.665) (end 183.62 126.345) (width 0.2) (layer "F.Cu") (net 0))
 (segment (start 136.62 87.005) (end 145.52 78.105) (width 0.2) (layer "F.Cu") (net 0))
 (segment (start 181.08 113.665) (end 182.35 114.935) (width 0.2) (layer "F.Cu") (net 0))
 (segment (start 177.24 113.665) (end 181.08 113.665) (width 0.2) (layer "F.Cu") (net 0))
 (segment (start 151.91 87.005) (end 140.465 98.45) (width 0.2) (layer "F.Cu") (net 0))
 (segment (start 179.81 116.205) (end 181.08 117.475) (width 0.2) (layer "F.Cu") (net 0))
 (segment (start 175.98 109.865) (end 177.24 111.125) (width 0.2) (layer "F.Cu") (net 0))
 (segment (start 148.06 70.485) (end 167.08 70.485) (width 0.2) (layer "F.Cu") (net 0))
 (segment (start 177.24 116.205) (end 179.81 116.205) (width 0.2) (layer "F.Cu") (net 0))
 (segment (start 117.56 120.025) (end 120.11 120.025) (width 0.2) (layer "F.Cu") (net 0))
 (segment (start 181.08 111.125) (end 183.62 113.665) (width 0.2) (layer "F.Cu") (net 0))
 (segment (start 121.39 120.015) (end 132.795 108.61) (width 0.2) (layer "F.Cu") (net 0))
 (segment (start 183.62 126.345) (end 186.16 128.885) (width 0.2) (layer "F.Cu") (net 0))
 (segment (start 136.62 94.625) (end 145.52 85.725) (width 0.2) (layer "F.Cu") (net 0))
 (segment (start 117.56 87.005) (end 136.62 87.005) (width 0.2) (layer "F.Cu") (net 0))
 (segment (start 136.62 92.085) (end 145.52 83.185) (width 0.2) (layer "F.Cu") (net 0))
 (segment (start 118.86 104.785) (end 117.56 104.785) (width 0.2) (layer "B.Cu") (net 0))
 (segment (start 125.2 111.125) (end 118.86 104.785) (width 0.2) (layer "B.Cu") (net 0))
 (segment (start 173.46 108.585) (end 173.46 116.205) (width 0.2) (layer "B.Cu") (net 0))
 (segment (start 122.66 128.905) (end 125.2 126.365) (width 0.2) (layer "B.Cu") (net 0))
 (segment (start 117.56 114.945) (end 118.86 114.945) (width 0.2) (layer "B.Cu") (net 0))
 (segment (start 146.79 128.905) (end 146.79 125.095) (width 0.2) (layer "B.Cu") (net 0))
 (segment (start 123.93 112.395) (end 118.86 107.325) (width 0.2) (layer "B.Cu") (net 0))
 (segment (start 118.84 109.865) (end 118.85 109.855) (width 0.2) (layer "B.Cu") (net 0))
 (segment (start 118.86 112.405) (end 117.56 112.405) (width 0.2) (layer "B.Cu") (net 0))
 (segment (start 120.12 128.905) (end 123.93 125.095) (width 0.2) (layer "B.Cu") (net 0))
 (segment (start 175.98 120.025) (end 172.19 116.235) (width 0.2) (layer "B.Cu") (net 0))
 (segment (start 117.56 99.705) (end 118.84 99.705) (width 0.2) (layer "B.Cu") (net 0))
 (segment (start 118.86 102.245) (end 117.56 102.245) (width 0.2) (layer "B.Cu") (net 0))
 (segment (start 123.93 125.095) (end 123.93 112.395) (width 0.2) (layer "B.Cu") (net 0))
 (segment (start 120.12 121.285) (end 112.5 128.905) (width 0.2) (layer "B.Cu") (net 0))
 (segment (start 153.14 128.905) (end 123.93 99.695) (width 0.2) (layer "B.Cu") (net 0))
 (segment (start 136.63 84.455) (end 145.52 75.565) (width 0.2) (layer "B.Cu") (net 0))
 (segment (start 146.79 125.095) (end 121.39 99.695) (width 0.2) (layer "B.Cu") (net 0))
 (segment (start 123.93 99.695) (end 123.93 80.675) (width 0.2) (layer "B.Cu") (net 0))
 (segment (start 173.46 116.205) (end 174.74 117.485) (width 0.2) (layer "B.Cu") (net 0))
 (segment (start 125.2 128.905) (end 126.47 127.635) (width 0.2) (layer "B.Cu") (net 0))
 (segment (start 126.47 127.635) (end 126.47 109.855) (width 0.2) (layer "B.Cu") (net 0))
 (segment (start 122.66 113.665) (end 122.66 123.825) (width 0.2) (layer "B.Cu") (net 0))
 (segment (start 118.85 99.695) (end 140.44 121.285) (width 0.2) (layer "B.Cu") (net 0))
 (segment (start 175.98 107.325) (end 174.74 107.325) (width 0.2) (layer "B.Cu") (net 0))
 (segment (start 172.19 109.855) (end 148.06 85.725) (width 0.2) (layer "B.Cu") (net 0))
 (segment (start 121.39 99.695) (end 121.39 80.675) (width 0.2) (layer "B.Cu") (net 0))
 (segment (start 121.39 80.675) (end 117.56 76.845) (width 0.2) (layer "B.Cu") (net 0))
 (segment (start 140.465 103.53) (end 136.63 99.695) (width 0.2) (layer "B.Cu") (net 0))
 (segment (start 174.74 107.325) (end 148.06 80.645) (width 0.2) (layer "B.Cu") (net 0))
 (segment (start 126.47 109.855) (end 118.86 102.245) (width 0.2) (layer "B.Cu") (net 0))
 (segment (start 118.85 109.855) (end 122.66 113.665) (width 0.2) (layer "B.Cu") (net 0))
 (segment (start 125.2 126.365) (end 125.2 111.125) (width 0.2) (layer "B.Cu") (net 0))
 (segment (start 174.74 117.485) (end 175.98 117.485) (width 0.2) (layer "B.Cu") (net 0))
 (segment (start 123.93 80.675) (end 117.56 74.305) (width 0.2) (layer "B.Cu") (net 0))
 (segment (start 115.04 128.905) (end 121.39 122.555) (width 0.2) (layer "B.Cu") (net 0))
 (segment (start 121.39 122.555) (end 121.39 114.935) (width 0.2) (layer "B.Cu") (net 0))
 (segment (start 118.84 99.705) (end 118.85 99.695) (width 0.2) (layer "B.Cu") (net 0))
 (segment (start 148.06 83.185) (end 173.46 108.585) (width 0.2) (layer "B.Cu") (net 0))
 (segment (start 118.86 107.325) (end 117.56 107.325) (width 0.2) (layer "B.Cu") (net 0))
 (segment (start 172.19 116.235) (end 172.19 109.855) (width 0.2) (layer "B.Cu") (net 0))
 (segment (start 136.63 99.695) (end 136.63 84.455) (width 0.2) (layer "B.Cu") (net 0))
 (segment (start 121.39 114.935) (end 118.86 112.405) (width 0.2) (layer "B.Cu") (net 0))
 (segment (start 122.66 123.825) (end 117.58 128.905) (width 0.2) (layer "B.Cu") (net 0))
 (segment (start 118.86 114.945) (end 120.12 116.205) (width 0.2) (layer "B.Cu") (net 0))
 (segment (start 140.44 121.285) (end 140.44 128.905) (width 0.2) (layer "B.Cu") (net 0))
 (segment (start 117.56 109.865) (end 118.84 109.865) (width 0.2) (layer "B.Cu") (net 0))
 (segment (start 120.12 116.205) (end 120.12 121.285) (width 0.2) (layer "B.Cu") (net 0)))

